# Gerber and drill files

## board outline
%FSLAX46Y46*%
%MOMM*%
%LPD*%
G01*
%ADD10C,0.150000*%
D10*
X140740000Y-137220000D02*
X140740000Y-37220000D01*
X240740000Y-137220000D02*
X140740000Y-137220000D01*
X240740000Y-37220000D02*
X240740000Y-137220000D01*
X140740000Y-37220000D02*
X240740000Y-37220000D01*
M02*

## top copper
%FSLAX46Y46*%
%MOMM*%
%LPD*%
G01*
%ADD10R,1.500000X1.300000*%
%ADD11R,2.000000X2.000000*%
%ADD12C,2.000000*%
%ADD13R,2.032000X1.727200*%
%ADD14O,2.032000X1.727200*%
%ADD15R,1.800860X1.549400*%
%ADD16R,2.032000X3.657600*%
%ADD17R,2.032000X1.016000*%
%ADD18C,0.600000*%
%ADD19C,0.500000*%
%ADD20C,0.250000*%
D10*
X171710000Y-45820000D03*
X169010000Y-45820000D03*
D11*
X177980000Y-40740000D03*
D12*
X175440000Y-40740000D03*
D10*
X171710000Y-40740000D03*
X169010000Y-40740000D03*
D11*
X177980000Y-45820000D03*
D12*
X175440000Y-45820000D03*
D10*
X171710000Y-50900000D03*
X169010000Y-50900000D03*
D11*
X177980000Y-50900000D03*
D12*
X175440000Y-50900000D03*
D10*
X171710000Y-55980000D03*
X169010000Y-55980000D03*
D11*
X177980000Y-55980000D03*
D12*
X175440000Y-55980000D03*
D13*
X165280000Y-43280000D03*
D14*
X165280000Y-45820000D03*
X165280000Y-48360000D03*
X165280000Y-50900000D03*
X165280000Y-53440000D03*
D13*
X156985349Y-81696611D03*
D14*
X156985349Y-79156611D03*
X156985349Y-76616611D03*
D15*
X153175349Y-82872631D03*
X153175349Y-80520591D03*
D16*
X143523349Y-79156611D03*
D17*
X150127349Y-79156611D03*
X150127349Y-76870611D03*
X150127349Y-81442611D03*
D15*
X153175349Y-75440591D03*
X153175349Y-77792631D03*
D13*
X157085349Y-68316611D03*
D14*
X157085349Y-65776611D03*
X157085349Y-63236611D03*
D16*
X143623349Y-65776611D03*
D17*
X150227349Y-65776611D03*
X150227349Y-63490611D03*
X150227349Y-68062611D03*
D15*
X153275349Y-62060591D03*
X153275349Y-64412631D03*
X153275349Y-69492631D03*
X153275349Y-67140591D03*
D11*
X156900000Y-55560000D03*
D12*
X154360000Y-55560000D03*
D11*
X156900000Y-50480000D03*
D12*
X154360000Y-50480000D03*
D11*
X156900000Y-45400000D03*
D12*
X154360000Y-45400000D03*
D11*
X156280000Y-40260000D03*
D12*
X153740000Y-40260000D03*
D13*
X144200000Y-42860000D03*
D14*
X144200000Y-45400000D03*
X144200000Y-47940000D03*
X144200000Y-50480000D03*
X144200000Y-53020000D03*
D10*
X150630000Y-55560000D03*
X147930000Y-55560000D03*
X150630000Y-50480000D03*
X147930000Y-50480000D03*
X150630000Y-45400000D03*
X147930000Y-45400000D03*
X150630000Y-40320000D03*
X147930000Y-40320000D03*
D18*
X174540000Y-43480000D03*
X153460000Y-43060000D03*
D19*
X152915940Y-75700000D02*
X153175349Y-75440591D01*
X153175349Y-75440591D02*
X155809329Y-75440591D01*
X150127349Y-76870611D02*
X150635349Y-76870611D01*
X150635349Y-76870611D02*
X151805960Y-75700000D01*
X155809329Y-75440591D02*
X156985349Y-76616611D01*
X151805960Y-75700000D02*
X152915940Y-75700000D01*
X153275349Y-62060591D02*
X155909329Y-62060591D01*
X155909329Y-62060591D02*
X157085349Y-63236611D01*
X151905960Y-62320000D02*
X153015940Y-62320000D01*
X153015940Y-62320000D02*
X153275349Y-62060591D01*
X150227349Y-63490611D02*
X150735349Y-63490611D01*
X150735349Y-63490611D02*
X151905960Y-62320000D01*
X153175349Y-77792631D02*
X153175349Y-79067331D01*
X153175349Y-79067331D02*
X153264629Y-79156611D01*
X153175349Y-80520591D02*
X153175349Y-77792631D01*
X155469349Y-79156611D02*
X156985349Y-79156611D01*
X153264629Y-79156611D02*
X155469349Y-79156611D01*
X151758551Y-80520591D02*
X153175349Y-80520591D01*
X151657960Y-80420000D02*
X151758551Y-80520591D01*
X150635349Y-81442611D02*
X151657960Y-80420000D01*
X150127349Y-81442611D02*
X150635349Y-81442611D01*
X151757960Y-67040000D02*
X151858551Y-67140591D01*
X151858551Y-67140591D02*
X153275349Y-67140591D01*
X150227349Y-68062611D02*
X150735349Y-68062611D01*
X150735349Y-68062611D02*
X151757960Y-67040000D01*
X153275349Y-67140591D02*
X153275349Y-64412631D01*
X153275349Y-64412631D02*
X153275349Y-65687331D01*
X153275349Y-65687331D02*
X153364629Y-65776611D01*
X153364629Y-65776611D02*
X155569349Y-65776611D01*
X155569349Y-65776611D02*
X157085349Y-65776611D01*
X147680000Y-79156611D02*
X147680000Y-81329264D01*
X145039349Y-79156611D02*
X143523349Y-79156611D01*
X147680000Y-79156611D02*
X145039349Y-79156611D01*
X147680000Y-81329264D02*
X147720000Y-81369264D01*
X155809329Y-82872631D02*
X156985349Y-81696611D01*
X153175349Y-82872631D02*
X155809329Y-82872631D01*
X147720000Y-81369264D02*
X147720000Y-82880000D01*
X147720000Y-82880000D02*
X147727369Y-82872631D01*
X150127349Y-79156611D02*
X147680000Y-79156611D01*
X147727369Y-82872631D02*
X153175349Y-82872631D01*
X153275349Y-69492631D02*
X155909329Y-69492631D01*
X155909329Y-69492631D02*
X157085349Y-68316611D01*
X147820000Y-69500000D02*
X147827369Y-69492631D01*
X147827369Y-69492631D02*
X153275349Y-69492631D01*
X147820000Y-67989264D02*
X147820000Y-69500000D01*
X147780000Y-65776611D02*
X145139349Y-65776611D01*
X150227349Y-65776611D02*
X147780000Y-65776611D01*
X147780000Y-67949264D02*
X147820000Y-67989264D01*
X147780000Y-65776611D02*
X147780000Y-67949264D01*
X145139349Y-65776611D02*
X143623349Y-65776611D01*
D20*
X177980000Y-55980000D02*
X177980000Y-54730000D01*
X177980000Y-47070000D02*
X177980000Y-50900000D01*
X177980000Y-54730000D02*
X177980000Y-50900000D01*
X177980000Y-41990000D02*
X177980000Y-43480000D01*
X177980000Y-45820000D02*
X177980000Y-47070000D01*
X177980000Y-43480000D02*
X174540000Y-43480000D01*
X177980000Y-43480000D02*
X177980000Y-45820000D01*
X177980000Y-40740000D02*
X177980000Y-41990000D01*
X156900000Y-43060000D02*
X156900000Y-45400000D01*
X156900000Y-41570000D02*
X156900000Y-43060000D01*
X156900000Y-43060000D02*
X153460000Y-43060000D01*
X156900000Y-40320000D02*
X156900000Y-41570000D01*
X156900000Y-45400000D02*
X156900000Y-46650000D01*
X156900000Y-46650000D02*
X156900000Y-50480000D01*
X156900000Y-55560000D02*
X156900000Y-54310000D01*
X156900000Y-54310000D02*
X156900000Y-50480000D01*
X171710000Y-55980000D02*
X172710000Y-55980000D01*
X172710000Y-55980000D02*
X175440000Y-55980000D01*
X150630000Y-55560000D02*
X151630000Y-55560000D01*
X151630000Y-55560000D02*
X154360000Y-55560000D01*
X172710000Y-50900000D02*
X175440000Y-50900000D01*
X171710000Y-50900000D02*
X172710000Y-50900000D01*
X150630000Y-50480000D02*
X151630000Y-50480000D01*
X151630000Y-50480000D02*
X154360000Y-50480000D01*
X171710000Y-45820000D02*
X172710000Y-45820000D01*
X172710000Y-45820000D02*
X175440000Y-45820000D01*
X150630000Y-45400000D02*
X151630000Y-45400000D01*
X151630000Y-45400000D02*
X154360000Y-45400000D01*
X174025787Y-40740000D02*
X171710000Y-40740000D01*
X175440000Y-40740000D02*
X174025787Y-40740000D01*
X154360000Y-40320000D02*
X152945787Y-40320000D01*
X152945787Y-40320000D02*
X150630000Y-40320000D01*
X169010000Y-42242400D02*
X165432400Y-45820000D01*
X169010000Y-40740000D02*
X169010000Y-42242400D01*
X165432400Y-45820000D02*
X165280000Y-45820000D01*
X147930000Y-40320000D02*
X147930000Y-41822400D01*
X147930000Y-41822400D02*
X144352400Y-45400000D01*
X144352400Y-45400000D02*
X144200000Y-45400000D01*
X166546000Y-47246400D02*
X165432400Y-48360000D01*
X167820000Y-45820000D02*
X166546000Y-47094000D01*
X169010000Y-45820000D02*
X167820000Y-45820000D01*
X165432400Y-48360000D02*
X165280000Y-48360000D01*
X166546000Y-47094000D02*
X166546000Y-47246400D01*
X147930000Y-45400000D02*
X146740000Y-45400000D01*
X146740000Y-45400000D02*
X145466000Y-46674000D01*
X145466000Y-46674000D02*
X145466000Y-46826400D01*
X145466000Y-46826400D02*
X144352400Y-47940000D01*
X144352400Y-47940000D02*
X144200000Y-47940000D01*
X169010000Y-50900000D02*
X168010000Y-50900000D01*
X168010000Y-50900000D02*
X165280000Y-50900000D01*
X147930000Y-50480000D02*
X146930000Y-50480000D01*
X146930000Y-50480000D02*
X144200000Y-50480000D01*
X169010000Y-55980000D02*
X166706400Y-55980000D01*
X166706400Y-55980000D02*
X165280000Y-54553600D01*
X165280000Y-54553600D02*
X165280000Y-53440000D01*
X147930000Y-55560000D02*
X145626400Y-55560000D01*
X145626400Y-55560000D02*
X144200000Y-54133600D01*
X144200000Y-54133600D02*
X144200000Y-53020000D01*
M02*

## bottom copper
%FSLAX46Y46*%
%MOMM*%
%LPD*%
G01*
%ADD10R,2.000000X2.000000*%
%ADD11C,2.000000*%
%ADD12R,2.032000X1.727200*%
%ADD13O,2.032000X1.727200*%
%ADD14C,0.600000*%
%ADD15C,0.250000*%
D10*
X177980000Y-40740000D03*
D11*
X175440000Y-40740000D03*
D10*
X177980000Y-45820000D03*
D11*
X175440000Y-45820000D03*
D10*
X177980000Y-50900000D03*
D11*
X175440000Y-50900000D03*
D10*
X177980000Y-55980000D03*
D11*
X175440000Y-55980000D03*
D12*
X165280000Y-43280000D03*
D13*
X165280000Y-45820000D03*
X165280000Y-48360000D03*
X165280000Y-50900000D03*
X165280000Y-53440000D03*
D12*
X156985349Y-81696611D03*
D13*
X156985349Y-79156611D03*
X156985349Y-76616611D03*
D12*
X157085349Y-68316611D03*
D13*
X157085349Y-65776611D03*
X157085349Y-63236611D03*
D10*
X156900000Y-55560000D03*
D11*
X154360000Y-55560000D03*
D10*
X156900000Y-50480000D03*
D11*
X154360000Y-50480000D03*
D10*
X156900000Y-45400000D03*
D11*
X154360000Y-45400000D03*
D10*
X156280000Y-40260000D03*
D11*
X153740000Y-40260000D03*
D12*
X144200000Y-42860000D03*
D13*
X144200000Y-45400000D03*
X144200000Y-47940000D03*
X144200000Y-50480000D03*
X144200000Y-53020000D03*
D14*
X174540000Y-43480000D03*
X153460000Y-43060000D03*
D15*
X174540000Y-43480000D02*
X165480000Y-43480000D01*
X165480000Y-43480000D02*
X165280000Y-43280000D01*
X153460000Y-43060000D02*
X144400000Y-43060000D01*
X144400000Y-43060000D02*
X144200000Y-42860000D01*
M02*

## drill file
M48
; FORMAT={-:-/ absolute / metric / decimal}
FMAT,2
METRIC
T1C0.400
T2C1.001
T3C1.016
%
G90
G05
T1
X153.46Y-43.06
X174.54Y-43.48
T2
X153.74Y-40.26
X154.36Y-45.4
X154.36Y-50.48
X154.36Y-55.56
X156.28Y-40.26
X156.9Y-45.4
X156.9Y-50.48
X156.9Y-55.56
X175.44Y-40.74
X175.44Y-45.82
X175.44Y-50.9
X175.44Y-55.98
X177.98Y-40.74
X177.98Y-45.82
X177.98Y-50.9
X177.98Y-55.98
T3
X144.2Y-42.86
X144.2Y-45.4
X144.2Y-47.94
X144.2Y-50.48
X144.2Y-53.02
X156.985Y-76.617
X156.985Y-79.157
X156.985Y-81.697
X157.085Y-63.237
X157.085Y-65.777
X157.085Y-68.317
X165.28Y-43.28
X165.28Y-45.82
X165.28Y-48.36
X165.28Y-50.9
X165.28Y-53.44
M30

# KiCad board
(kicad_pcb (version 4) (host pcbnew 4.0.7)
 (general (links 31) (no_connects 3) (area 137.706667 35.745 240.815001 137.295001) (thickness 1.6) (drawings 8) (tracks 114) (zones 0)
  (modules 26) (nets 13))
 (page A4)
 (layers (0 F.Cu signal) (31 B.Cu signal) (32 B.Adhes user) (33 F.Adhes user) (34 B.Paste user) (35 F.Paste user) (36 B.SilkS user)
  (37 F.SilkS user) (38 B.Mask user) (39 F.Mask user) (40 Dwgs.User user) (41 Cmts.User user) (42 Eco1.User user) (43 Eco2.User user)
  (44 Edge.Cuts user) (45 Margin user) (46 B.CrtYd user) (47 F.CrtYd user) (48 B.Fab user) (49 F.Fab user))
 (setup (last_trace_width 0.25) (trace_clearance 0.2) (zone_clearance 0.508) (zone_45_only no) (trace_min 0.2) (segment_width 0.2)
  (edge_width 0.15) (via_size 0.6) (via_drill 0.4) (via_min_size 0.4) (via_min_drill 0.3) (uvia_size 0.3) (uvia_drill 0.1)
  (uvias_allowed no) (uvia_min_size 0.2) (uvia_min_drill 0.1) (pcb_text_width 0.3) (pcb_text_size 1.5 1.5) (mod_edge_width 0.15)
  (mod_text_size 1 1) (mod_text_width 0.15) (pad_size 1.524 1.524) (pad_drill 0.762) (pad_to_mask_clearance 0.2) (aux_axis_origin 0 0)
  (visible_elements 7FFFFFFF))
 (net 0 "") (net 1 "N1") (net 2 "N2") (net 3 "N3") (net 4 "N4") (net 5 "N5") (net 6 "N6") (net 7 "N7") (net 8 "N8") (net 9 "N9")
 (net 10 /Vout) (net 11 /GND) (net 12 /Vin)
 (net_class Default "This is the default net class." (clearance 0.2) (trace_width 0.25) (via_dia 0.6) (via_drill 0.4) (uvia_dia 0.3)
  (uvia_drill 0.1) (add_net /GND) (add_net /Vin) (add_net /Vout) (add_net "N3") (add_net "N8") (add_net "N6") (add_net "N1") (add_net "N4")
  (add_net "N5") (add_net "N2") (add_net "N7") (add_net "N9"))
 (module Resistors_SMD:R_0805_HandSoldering (layer F.Cu) (at 170.36 45.82 180)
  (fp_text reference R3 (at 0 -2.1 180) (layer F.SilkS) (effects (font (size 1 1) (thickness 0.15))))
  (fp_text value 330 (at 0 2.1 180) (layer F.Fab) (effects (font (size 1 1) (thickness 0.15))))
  (pad 1 smd rect (at -1.35 0 180) (size 1.5 1.3) (layers F.Cu F.Paste F.Mask) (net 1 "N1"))
  (pad 2 smd rect (at 1.35 0 180) (size 1.5 1.3) (layers F.Cu F.Paste F.Mask) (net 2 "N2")))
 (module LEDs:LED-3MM (layer F.Cu) (at 177.98 40.74 180)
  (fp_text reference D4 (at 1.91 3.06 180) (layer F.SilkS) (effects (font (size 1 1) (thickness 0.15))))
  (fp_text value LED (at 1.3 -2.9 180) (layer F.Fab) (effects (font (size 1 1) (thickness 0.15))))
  (pad 1 thru_hole rect (at 0 0 270) (size 2 2) (drill 1.00076) (layers *.Cu *.Mask F.SilkS) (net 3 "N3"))
  (pad 2 thru_hole circle (at 2.54 0 180) (size 2 2) (drill 1.00076) (layers *.Cu *.Mask F.SilkS) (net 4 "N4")))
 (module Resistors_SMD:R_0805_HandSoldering (layer F.Cu) (at 170.36 40.74 180)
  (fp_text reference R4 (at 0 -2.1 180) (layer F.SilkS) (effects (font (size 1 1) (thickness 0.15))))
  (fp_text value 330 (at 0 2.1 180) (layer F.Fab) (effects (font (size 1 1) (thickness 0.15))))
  (pad 1 smd rect (at -1.35 0 180) (size 1.5 1.3) (layers F.Cu F.Paste F.Mask) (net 4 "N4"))
  (pad 2 smd rect (at 1.35 0 180) (size 1.5 1.3) (layers F.Cu F.Paste F.Mask) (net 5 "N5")))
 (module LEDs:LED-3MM (layer F.Cu) (at 177.98 45.82 180)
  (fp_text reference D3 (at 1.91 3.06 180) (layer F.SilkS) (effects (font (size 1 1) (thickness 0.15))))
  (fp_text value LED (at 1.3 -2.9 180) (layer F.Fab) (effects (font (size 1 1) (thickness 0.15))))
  (pad 1 thru_hole rect (at 0 0 270) (size 2 2) (drill 1.00076) (layers *.Cu *.Mask F.SilkS) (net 3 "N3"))
  (pad 2 thru_hole circle (at 2.54 0 180) (size 2 2) (drill 1.00076) (layers *.Cu *.Mask F.SilkS) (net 1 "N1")))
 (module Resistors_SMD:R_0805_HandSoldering (layer F.Cu) (at 170.36 50.9 180)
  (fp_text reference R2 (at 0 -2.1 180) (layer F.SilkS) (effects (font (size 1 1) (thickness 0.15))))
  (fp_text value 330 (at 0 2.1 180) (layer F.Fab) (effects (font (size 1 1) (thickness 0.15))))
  (pad 1 smd rect (at -1.35 0 180) (size 1.5 1.3) (layers F.Cu F.Paste F.Mask) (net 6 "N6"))
  (pad 2 smd rect (at 1.35 0 180) (size 1.5 1.3) (layers F.Cu F.Paste F.Mask) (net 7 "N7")))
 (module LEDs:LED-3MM (layer F.Cu) (at 177.98 50.9 180)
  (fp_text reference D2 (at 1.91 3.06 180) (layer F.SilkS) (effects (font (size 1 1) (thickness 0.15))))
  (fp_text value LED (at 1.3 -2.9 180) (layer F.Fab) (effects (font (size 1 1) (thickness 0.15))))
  (pad 1 thru_hole rect (at 0 0 270) (size 2 2) (drill 1.00076) (layers *.Cu *.Mask F.SilkS) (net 3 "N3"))
  (pad 2 thru_hole circle (at 2.54 0 180) (size 2 2) (drill 1.00076) (layers *.Cu *.Mask F.SilkS) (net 6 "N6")))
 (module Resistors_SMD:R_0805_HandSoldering (layer F.Cu) (at 170.36 55.98 180)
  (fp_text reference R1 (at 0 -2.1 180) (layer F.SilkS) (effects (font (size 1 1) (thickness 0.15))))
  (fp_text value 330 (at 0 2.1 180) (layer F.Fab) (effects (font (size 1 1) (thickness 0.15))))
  (pad 1 smd rect (at -1.35 0 180) (size 1.5 1.3) (layers F.Cu F.Paste F.Mask) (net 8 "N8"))
  (pad 2 smd rect (at 1.35 0 180) (size 1.5 1.3) (layers F.Cu F.Paste F.Mask) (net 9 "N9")))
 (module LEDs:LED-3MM (layer F.Cu) (at 177.98 55.98 180)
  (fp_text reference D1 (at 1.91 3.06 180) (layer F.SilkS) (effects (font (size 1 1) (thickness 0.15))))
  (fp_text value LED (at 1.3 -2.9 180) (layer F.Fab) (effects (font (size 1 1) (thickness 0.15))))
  (pad 1 thru_hole rect (at 0 0 270) (size 2 2) (drill 1.00076) (layers *.Cu *.Mask F.SilkS) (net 3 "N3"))
  (pad 2 thru_hole circle (at 2.54 0 180) (size 2 2) (drill 1.00076) (layers *.Cu *.Mask F.SilkS) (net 8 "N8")))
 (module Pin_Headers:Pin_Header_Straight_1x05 (layer F.Cu) (at 165.28 43.28)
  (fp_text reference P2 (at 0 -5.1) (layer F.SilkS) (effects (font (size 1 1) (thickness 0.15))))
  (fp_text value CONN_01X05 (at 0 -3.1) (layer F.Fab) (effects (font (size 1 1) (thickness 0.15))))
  (pad 1 thru_hole rect (at 0 0) (size 2.032 1.7272) (drill 1.016) (layers *.Cu *.Mask F.SilkS) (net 3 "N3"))
  (pad 2 thru_hole oval (at 0 2.54) (size 2.032 1.7272) (drill 1.016) (layers *.Cu *.Mask F.SilkS) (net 5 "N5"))
  (pad 3 thru_hole oval (at 0 5.08) (size 2.032 1.7272) (drill 1.016) (layers *.Cu *.Mask F.SilkS) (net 2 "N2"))
  (pad 4 thru_hole oval (at 0 7.62) (size 2.032 1.7272) (drill 1.016) (layers *.Cu *.Mask F.SilkS) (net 7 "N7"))
  (pad 5 thru_hole oval (at 0 10.16) (size 2.032 1.7272) (drill 1.016) (layers *.Cu *.Mask F.SilkS) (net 9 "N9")))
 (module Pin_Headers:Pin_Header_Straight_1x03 (layer F.Cu) (at 156.985349 81.696611 180)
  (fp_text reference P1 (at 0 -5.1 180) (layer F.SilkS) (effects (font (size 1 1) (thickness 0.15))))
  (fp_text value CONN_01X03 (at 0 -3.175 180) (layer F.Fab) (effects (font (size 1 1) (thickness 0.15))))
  (pad 1 thru_hole rect (at 0 0 180) (size 2.032 1.7272) (drill 1.016) (layers *.Cu *.Mask F.SilkS) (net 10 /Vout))
  (pad 2 thru_hole oval (at 0 2.54 180) (size 2.032 1.7272) (drill 1.016) (layers *.Cu *.Mask F.SilkS) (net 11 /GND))
  (pad 3 thru_hole oval (at 0 5.08 180) (size 2.032 1.7272) (drill 1.016) (layers *.Cu *.Mask F.SilkS) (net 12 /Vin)))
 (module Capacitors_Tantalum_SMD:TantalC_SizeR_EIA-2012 (layer F.Cu) (at 153.175349 81.696611 270)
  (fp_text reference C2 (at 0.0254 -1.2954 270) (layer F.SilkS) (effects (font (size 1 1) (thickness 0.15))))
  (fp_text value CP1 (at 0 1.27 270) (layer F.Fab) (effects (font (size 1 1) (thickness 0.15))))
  (pad 1 smd rect (at 1.17602 0 270) (size 1.5494 1.80086) (layers F.Cu F.Paste F.Mask) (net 10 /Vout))
  (pad 2 smd rect (at -1.17602 0 270) (size 1.5494 1.80086) (layers F.Cu F.Paste F.Mask) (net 11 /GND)))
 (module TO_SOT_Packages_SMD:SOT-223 (layer F.Cu) (at 146.825349 79.156611 90)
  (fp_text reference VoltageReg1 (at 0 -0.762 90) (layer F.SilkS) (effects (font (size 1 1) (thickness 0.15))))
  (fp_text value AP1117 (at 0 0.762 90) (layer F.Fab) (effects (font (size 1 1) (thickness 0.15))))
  (pad 4 smd rect (at 0 -3.302 90) (size 3.6576 2.032) (layers F.Cu F.Paste F.Mask) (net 10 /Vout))
  (pad 2 smd rect (at 0 3.302 90) (size 1.016 2.032) (layers F.Cu F.Paste F.Mask) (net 10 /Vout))
  (pad 3 smd rect (at 2.286 3.302 90) (size 1.016 2.032) (layers F.Cu F.Paste F.Mask) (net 12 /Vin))
  (pad 1 smd rect (at -2.286 3.302 90) (size 1.016 2.032) (layers F.Cu F.Paste F.Mask) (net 11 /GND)))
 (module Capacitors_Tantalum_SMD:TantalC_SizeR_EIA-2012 (layer F.Cu) (at 153.175349 76.616611 90)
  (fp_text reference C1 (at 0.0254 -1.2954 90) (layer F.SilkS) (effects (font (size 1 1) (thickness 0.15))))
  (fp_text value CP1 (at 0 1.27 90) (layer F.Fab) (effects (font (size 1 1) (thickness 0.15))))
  (pad 1 smd rect (at 1.17602 0 90) (size 1.5494 1.80086) (layers F.Cu F.Paste F.Mask) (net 12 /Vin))
  (pad 2 smd rect (at -1.17602 0 90) (size 1.5494 1.80086) (layers F.Cu F.Paste F.Mask) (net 11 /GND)))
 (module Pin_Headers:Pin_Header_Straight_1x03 (layer F.Cu) (at 157.085349 68.316611 180)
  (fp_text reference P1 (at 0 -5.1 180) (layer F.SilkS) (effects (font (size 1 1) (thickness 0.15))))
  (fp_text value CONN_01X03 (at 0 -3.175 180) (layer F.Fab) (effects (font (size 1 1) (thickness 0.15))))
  (pad 1 thru_hole rect (at 0 0 180) (size 2.032 1.7272) (drill 1.016) (layers *.Cu *.Mask F.SilkS) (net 10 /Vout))
  (pad 2 thru_hole oval (at 0 2.54 180) (size 2.032 1.7272) (drill 1.016) (layers *.Cu *.Mask F.SilkS) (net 11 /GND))
  (pad 3 thru_hole oval (at 0 5.08 180) (size 2.032 1.7272) (drill 1.016) (layers *.Cu *.Mask F.SilkS) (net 12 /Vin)))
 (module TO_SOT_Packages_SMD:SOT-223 (layer F.Cu) (at 146.925349 65.776611 90)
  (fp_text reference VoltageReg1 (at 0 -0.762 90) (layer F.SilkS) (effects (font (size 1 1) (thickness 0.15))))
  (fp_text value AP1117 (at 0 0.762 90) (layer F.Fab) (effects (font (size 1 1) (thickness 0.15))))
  (pad 4 smd rect (at 0 -3.302 90) (size 3.6576 2.032) (layers F.Cu F.Paste F.Mask) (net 10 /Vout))
  (pad 2 smd rect (at 0 3.302 90) (size 1.016 2.032) (layers F.Cu F.Paste F.Mask) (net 10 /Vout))
  (pad 3 smd rect (at 2.286 3.302 90) (size 1.016 2.032) (layers F.Cu F.Paste F.Mask) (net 12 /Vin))
  (pad 1 smd rect (at -2.286 3.302 90) (size 1.016 2.032) (layers F.Cu F.Paste F.Mask) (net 11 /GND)))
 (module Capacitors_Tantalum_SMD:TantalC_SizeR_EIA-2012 (layer F.Cu) (at 153.275349 63.236611 90)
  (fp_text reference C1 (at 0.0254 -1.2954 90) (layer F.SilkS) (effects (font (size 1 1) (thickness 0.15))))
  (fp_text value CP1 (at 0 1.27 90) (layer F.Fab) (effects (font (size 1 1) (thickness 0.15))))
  (pad 1 smd rect (at 1.17602 0 90) (size 1.5494 1.80086) (layers F.Cu F.Paste F.Mask) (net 12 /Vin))
  (pad 2 smd rect (at -1.17602 0 90) (size 1.5494 1.80086) (layers F.Cu F.Paste F.Mask) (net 11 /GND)))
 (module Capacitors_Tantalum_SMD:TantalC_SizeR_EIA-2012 (layer F.Cu) (at 153.275349 68.316611 270)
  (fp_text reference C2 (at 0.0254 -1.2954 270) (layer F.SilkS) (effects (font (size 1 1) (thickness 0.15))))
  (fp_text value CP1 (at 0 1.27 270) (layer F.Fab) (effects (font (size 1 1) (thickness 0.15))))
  (pad 1 smd rect (at 1.17602 0 270) (size 1.5494 1.80086) (layers F.Cu F.Paste F.Mask) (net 10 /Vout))
  (pad 2 smd rect (at -1.17602 0 270) (size 1.5494 1.80086) (layers F.Cu F.Paste F.Mask) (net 11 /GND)))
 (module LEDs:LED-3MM (layer F.Cu) (at 156.9 55.56 180)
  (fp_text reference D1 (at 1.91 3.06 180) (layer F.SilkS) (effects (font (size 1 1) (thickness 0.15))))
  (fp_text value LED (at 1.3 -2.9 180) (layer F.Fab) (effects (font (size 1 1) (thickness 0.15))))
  (pad 1 thru_hole rect (at 0 0 270) (size 2 2) (drill 1.00076) (layers *.Cu *.Mask F.SilkS) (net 3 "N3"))
  (pad 2 thru_hole circle (at 2.54 0 180) (size 2 2) (drill 1.00076) (layers *.Cu *.Mask F.SilkS) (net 8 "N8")))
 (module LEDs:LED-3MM (layer F.Cu) (at 156.9 50.48 180)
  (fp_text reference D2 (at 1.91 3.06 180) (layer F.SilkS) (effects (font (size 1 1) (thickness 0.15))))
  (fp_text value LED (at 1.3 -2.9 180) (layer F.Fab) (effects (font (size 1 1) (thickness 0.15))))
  (pad 1 thru_hole rect (at 0 0 270) (size 2 2) (drill 1.00076) (layers *.Cu *.Mask F.SilkS) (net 3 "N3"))
  (pad 2 thru_hole circle (at 2.54 0 180) (size 2 2) (drill 1.00076) (layers *.Cu *.Mask F.SilkS) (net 6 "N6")))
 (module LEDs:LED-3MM (layer F.Cu) (at 156.9 45.4 180)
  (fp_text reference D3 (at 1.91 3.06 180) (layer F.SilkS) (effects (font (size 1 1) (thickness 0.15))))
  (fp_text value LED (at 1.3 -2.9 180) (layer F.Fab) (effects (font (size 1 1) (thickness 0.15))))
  (pad 1 thru_hole rect (at 0 0 270) (size 2 2) (drill 1.00076) (layers *.Cu *.Mask F.SilkS) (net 3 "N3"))
  (pad 2 thru_hole circle (at 2.54 0 180) (size 2 2) (drill 1.00076) (layers *.Cu *.Mask F.SilkS) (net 1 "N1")))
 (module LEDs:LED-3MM (layer F.Cu) (at 156.28 40.26 180)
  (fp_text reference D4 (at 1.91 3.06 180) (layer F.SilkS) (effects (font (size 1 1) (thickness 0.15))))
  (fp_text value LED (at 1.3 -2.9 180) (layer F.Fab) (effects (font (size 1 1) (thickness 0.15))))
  (pad 1 thru_hole rect (at 0 0 270) (size 2 2) (drill 1.00076) (layers *.Cu *.Mask F.SilkS) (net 3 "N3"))
  (pad 2 thru_hole circle (at 2.54 0 180) (size 2 2) (drill 1.00076) (layers *.Cu *.Mask F.SilkS) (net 4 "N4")))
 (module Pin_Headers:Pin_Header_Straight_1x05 (layer F.Cu) (at 144.2 42.86)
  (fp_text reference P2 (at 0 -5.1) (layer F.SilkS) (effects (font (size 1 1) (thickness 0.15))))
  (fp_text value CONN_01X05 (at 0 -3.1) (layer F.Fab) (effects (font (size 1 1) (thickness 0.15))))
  (pad 1 thru_hole rect (at 0 0) (size 2.032 1.7272) (drill 1.016) (layers *.Cu *.Mask F.SilkS) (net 3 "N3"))
  (pad 2 thru_hole oval (at 0 2.54) (size 2.032 1.7272) (drill 1.016) (layers *.Cu *.Mask F.SilkS) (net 5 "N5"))
  (pad 3 thru_hole oval (at 0 5.08) (size 2.032 1.7272) (drill 1.016) (layers *.Cu *.Mask F.SilkS) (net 2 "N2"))
  (pad 4 thru_hole oval (at 0 7.62) (size 2.032 1.7272) (drill 1.016) (layers *.Cu *.Mask F.SilkS) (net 7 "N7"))
  (pad 5 thru_hole oval (at 0 10.16) (size 2.032 1.7272) (drill 1.016) (layers *.Cu *.Mask F.SilkS) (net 9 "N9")))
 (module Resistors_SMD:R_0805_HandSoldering (layer F.Cu) (at 149.28 55.56 180)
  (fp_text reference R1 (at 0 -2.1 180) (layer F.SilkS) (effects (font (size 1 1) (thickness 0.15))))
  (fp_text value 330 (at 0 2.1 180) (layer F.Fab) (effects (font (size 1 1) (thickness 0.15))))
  (pad 1 smd rect (at -1.35 0 180) (size 1.5 1.3) (layers F.Cu F.Paste F.Mask) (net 8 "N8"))
  (pad 2 smd rect (at 1.35 0 180) (size 1.5 1.3) (layers F.Cu F.Paste F.Mask) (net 9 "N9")))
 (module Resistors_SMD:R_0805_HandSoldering (layer F.Cu) (at 149.28 50.48 180)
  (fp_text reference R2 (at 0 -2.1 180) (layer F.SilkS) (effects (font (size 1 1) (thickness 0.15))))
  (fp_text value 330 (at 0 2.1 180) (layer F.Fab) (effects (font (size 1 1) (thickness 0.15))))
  (pad 1 smd rect (at -1.35 0 180) (size 1.5 1.3) (layers F.Cu F.Paste F.Mask) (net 6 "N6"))
  (pad 2 smd rect (at 1.35 0 180) (size 1.5 1.3) (layers F.Cu F.Paste F.Mask) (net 7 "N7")))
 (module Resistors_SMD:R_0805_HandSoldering (layer F.Cu) (at 149.28 45.4 180)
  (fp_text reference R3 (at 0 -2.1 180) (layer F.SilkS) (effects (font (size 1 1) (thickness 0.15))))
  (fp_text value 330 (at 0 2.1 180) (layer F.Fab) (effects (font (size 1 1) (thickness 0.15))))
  (pad 1 smd rect (at -1.35 0 180) (size 1.5 1.3) (layers F.Cu F.Paste F.Mask) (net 1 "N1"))
  (pad 2 smd rect (at 1.35 0 180) (size 1.5 1.3) (layers F.Cu F.Paste F.Mask) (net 2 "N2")))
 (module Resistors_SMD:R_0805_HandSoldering (layer F.Cu) (at 149.28 40.32 180)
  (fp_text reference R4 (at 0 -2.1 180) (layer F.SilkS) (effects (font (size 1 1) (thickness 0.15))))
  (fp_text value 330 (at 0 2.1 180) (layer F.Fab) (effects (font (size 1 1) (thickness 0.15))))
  (pad 1 smd rect (at -1.35 0 180) (size 1.5 1.3) (layers F.Cu F.Paste F.Mask) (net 4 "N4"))
  (pad 2 smd rect (at 1.35 0 180) (size 1.5 1.3) (layers F.Cu F.Paste F.Mask) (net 5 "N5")))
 (gr_line (start 140.74 137.22) (end 140.74 37.22) (layer Edge.Cuts) (width 0.15))
 (gr_line (start 240.74 137.22) (end 140.74 137.22) (layer Edge.Cuts) (width 0.15))
 (gr_line (start 240.74 37.22) (end 240.74 137.22) (layer Edge.Cuts) (width 0.15))
 (gr_line (start 140.74 37.22) (end 240.74 37.22) (layer Edge.Cuts) (width 0.15))
 (segment (start 152.91594 75.7) (end 153.175349 75.440591) (width 0.5) (layer F.Cu) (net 12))
 (segment (start 153.175349 75.440591) (end 155.809329 75.440591) (width 0.5) (layer F.Cu) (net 12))
 (segment (start 150.127349 76.870611) (end 150.635349 76.870611) (width 0.5) (layer F.Cu) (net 12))
 (segment (start 150.635349 76.870611) (end 151.80596 75.7) (width 0.5) (layer F.Cu) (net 12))
 (segment (start 155.809329 75.440591) (end 156.985349 76.616611) (width 0.5) (layer F.Cu) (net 12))
 (segment (start 151.80596 75.7) (end 152.91594 75.7) (width 0.5) (layer F.Cu) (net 12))
 (segment (start 153.275349 62.060591) (end 155.909329 62.060591) (width 0.5) (layer F.Cu) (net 12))
 (segment (start 155.909329 62.060591) (end 157.085349 63.236611) (width 0.5) (layer F.Cu) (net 12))
 (segment (start 151.90596 62.32) (end 153.01594 62.32) (width 0.5) (layer F.Cu) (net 12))
 (segment (start 153.01594 62.32) (end 153.275349 62.060591) (width 0.5) (layer F.Cu) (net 12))
 (segment (start 150.227349 63.490611) (end 150.735349 63.490611) (width 0.5) (layer F.Cu) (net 12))
 (segment (start 150.735349 63.490611) (end 151.90596 62.32) (width 0.5) (layer F.Cu) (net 12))
 (segment (start 153.175349 77.792631) (end 153.175349 79.067331) (width 0.5) (layer F.Cu) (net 11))
 (segment (start 153.175349 79.067331) (end 153.264629 79.156611) (width 0.5) (layer F.Cu) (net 11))
 (segment (start 153.175349 80.520591) (end 153.175349 77.792631) (width 0.5) (layer F.Cu) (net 11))
 (segment (start 155.469349 79.156611) (end 156.985349 79.156611) (width 0.5) (layer F.Cu) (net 11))
 (segment (start 153.264629 79.156611) (end 155.469349 79.156611) (width 0.5) (layer F.Cu) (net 11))
 (segment (start 151.758551 80.520591) (end 153.175349 80.520591) (width 0.5) (layer F.Cu) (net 11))
 (segment (start 151.65796 80.42) (end 151.758551 80.520591) (width 0.5) (layer F.Cu) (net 11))
 (segment (start 150.635349 81.442611) (end 151.65796 80.42) (width 0.5) (layer F.Cu) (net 11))
 (segment (start 150.127349 81.442611) (end 150.635349 81.442611) (width 0.5) (layer F.Cu) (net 11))
 (segment (start 151.75796 67.04) (end 151.858551 67.140591) (width 0.5) (layer F.Cu) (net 11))
 (segment (start 151.858551 67.140591) (end 153.275349 67.140591) (width 0.5) (layer F.Cu) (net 11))
 (segment (start 150.227349 68.062611) (end 150.735349 68.062611) (width 0.5) (layer F.Cu) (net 11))
 (segment (start 150.735349 68.062611) (end 151.75796 67.04) (width 0.5) (layer F.Cu) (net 11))
 (segment (start 153.275349 67.140591) (end 153.275349 64.412631) (width 0.5) (layer F.Cu) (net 11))
 (segment (start 153.275349 64.412631) (end 153.275349 65.687331) (width 0.5) (layer F.Cu) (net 11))
 (segment (start 153.275349 65.687331) (end 153.364629 65.776611) (width 0.5) (layer F.Cu) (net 11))
 (segment (start 153.364629 65.776611) (end 155.569349 65.776611) (width 0.5) (layer F.Cu) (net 11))
 (segment (start 155.569349 65.776611) (end 157.085349 65.776611) (width 0.5) (layer F.Cu) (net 11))
 (segment (start 147.68 79.156611) (end 147.68 81.329264) (width 0.5) (layer F.Cu) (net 10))
 (segment (start 145.039349 79.156611) (end 143.523349 79.156611) (width 0.5) (layer F.Cu) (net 10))
 (segment (start 147.68 79.156611) (end 145.039349 79.156611) (width 0.5) (layer F.Cu) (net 10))
 (segment (start 147.68 81.329264) (end 147.72 81.369264) (width 0.5) (layer F.Cu) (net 10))
 (segment (start 155.809329 82.872631) (end 156.985349 81.696611) (width 0.5) (layer F.Cu) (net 10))
 (segment (start 153.175349 82.872631) (end 155.809329 82.872631) (width 0.5) (layer F.Cu) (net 10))
 (segment (start 147.72 81.369264) (end 147.72 82.88) (width 0.5) (layer F.Cu) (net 10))
 (segment (start 147.72 82.88) (end 147.727369 82.872631) (width 0.5) (layer F.Cu) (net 10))
 (segment (start 150.127349 79.156611) (end 147.68 79.156611) (width 0.5) (layer F.Cu) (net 10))
 (segment (start 147.727369 82.872631) (end 153.175349 82.872631) (width 0.5) (layer F.Cu) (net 10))
 (segment (start 153.275349 69.492631) (end 155.909329 69.492631) (width 0.5) (layer F.Cu) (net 10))
 (segment (start 155.909329 69.492631) (end 157.085349 68.316611) (width 0.5) (layer F.Cu) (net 10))
 (segment (start 147.82 69.5) (end 147.827369 69.492631) (width 0.5) (layer F.Cu) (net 10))
 (segment (start 147.827369 69.492631) (end 153.275349 69.492631) (width 0.5) (layer F.Cu) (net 10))
 (segment (start 147.82 67.989264) (end 147.82 69.5) (width 0.5) (layer F.Cu) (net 10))
 (segment (start 147.78 65.776611) (end 145.139349 65.776611) (width 0.5) (layer F.Cu) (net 10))
 (segment (start 150.227349 65.776611) (end 147.78 65.776611) (width 0.5) (layer F.Cu) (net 10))
 (segment (start 147.78 67.949264) (end 147.82 67.989264) (width 0.5) (layer F.Cu) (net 10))
 (segment (start 147.78 65.776611) (end 147.78 67.949264) (width 0.5) (layer F.Cu) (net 10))
 (segment (start 145.139349 65.776611) (end 143.623349 65.776611) (width 0.5) (layer F.Cu) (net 10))
 (segment (start 174.54 43.48) (end 165.48 43.48) (width 0.25) (layer B.Cu) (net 3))
 (segment (start 165.48 43.48) (end 165.28 43.28) (width 0.25) (layer B.Cu) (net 3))
 (segment (start 177.98 55.98) (end 177.98 54.73) (width 0.25) (layer F.Cu) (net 3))
 (segment (start 177.98 47.07) (end 177.98 50.9) (width 0.25) (layer F.Cu) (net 3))
 (segment (start 177.98 54.73) (end 177.98 50.9) (width 0.25) (layer F.Cu) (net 3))
 (segment (start 177.98 41.99) (end 177.98 43.48) (width 0.25) (layer F.Cu) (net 3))
 (segment (start 177.98 45.82) (end 177.98 47.07) (width 0.25) (layer F.Cu) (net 3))
 (segment (start 177.98 43.48) (end 174.54 43.48) (width 0.25) (layer F.Cu) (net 3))
 (segment (start 177.98 43.48) (end 177.98 45.82) (width 0.25) (layer F.Cu) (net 3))
 (segment (start 177.98 40.74) (end 177.98 41.99) (width 0.25) (layer F.Cu) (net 3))
 (via (at 174.54 43.48) (size 0.6) (drill 0.4) (layers F.Cu B.Cu) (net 3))
 (segment (start 153.46 43.06) (end 144.4 43.06) (width 0.25) (layer B.Cu) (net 3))
 (segment (start 144.4 43.06) (end 144.2 42.86) (width 0.25) (layer B.Cu) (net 3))
 (via (at 153.46 43.06) (size 0.6) (drill 0.4) (layers F.Cu B.Cu) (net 3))
 (segment (start 156.9 43.06) (end 156.9 45.4) (width 0.25) (layer F.Cu) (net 3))
 (segment (start 156.9 41.57) (end 156.9 43.06) (width 0.25) (layer F.Cu) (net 3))
 (segment (start 156.9 43.06) (end 153.46 43.06) (width 0.25) (layer F.Cu) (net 3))
 (segment (start 156.9 40.32) (end 156.9 41.57) (width 0.25) (layer F.Cu) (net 3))
 (segment (start 156.9 45.4) (end 156.9 46.65) (width 0.25) (layer F.Cu) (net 3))
 (segment (start 156.9 46.65) (end 156.9 50.48) (width 0.25) (layer F.Cu) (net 3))
 (segment (start 156.9 55.56) (end 156.9 54.31) (width 0.25) (layer F.Cu) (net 3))
 (segment (start 156.9 54.31) (end 156.9 50.48) (width 0.25) (layer F.Cu) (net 3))
 (segment (start 171.71 55.98) (end 172.71 55.98) (width 0.25) (layer F.Cu) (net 8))
 (segment (start 172.71 55.98) (end 175.44 55.98) (width 0.25) (layer F.Cu) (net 8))
 (segment (start 150.63 55.56) (end 151.63 55.56) (width 0.25) (layer F.Cu) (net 8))
 (segment (start 151.63 55.56) (end 154.36 55.56) (width 0.25) (layer F.Cu) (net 8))
 (segment (start 172.71 50.9) (end 175.44 50.9) (width 0.25) (layer F.Cu) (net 6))
 (segment (start 171.71 50.9) (end 172.71 50.9) (width 0.25) (layer F.Cu) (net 6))
 (segment (start 150.63 50.48) (end 151.63 50.48) (width 0.25) (layer F.Cu) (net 6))
 (segment (start 151.63 50.48) (end 154.36 50.48) (width 0.25) (layer F.Cu) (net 6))
 (segment (start 171.71 45.82) (end 172.71 45.82) (width 0.25) (layer F.Cu) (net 1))
 (segment (start 172.71 45.82) (end 175.44 45.82) (width 0.25) (layer F.Cu) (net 1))
 (segment (start 150.63 45.4) (end 151.63 45.4) (width 0.25) (layer F.Cu) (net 1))
 (segment (start 151.63 45.4) (end 154.36 45.4) (width 0.25) (layer F.Cu) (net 1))
 (segment (start 174.025787 40.74) (end 171.71 40.74) (width 0.25) (layer F.Cu) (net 4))
 (segment (start 175.44 40.74) (end 174.025787 40.74) (width 0.25) (layer F.Cu) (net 4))
 (segment (start 154.36 40.32) (end 152.945787 40.32) (width 0.25) (layer F.Cu) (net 4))
 (segment (start 152.945787 40.32) (end 150.63 40.32) (width 0.25) (layer F.Cu) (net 4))
 (segment (start 169.01 42.2424) (end 165.4324 45.82) (width 0.25) (layer F.Cu) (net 5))
 (segment (start 169.01 40.74) (end 169.01 42.2424) (width 0.25) (layer F.Cu) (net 5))
 (segment (start 165.4324 45.82) (end 165.28 45.82) (width 0.25) (layer F.Cu) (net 5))
 (segment (start 147.93 40.32) (end 147.93 41.8224) (width 0.25) (layer F.Cu) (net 5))
 (segment (start 147.93 41.8224) (end 144.3524 45.4) (width 0.25) (layer F.Cu) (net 5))
 (segment (start 144.3524 45.4) (end 144.2 45.4) (width 0.25) (layer F.Cu) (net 5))
 (segment (start 166.546 47.2464) (end 165.4324 48.36) (width 0.25) (layer F.Cu) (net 2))
 (segment (start 167.82 45.82) (end 166.546 47.094) (width 0.25) (layer F.Cu) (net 2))
 (segment (start 169.01 45.82) (end 167.82 45.82) (width 0.25) (layer F.Cu) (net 2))
 (segment (start 165.4324 48.36) (end 165.28 48.36) (width 0.25) (layer F.Cu) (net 2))
 (segment (start 166.546 47.094) (end 166.546 47.2464) (width 0.25) (layer F.Cu) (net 2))
 (segment (start 147.93 45.4) (end 146.74 45.4) (width 0.25) (layer F.Cu) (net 2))
 (segment (start 146.74 45.4) (end 145.466 46.674) (width 0.25) (layer F.Cu) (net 2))
 (segment (start 145.466 46.674) (end 145.466 46.8264) (width 0.25) (layer F.Cu) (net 2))
 (segment (start 145.466 46.8264) (end 144.3524 47.94) (width 0.25) (layer F.Cu) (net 2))
 (segment (start 144.3524 47.94) (end 144.2 47.94) (width 0.25) (layer F.Cu) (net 2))
 (segment (start 169.01 50.9) (end 168.01 50.9) (width 0.25) (layer F.Cu) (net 7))
 (segment (start 168.01 50.9) (end 165.28 50.9) (width 0.25) (layer F.Cu) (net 7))
 (segment (start 147.93 50.48) (end 146.93 50.48) (width 0.25) (layer F.Cu) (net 7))
 (segment (start 146.93 50.48) (end 144.2 50.48) (width 0.25) (layer F.Cu) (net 7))
 (segment (start 169.01 55.98) (end 166.7064 55.98) (width 0.25) (layer F.Cu) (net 9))
 (segment (start 166.7064 55.98) (end 165.28 54.5536) (width 0.25) (layer F.Cu) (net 9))
 (segment (start 165.28 54.5536) (end 165.28 53.44) (width 0.25) (layer F.Cu) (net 9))
 (segment (start 147.93 55.56) (end 145.6264 55.56) (width 0.25) (layer F.Cu) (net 9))
 (segment (start 145.6264 55.56) (end 144.2 54.1336) (width 0.25) (layer F.Cu) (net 9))
 (segment (start 144.2 54.1336) (end 144.2 53.02) (width 0.25) (layer F.Cu) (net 9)))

